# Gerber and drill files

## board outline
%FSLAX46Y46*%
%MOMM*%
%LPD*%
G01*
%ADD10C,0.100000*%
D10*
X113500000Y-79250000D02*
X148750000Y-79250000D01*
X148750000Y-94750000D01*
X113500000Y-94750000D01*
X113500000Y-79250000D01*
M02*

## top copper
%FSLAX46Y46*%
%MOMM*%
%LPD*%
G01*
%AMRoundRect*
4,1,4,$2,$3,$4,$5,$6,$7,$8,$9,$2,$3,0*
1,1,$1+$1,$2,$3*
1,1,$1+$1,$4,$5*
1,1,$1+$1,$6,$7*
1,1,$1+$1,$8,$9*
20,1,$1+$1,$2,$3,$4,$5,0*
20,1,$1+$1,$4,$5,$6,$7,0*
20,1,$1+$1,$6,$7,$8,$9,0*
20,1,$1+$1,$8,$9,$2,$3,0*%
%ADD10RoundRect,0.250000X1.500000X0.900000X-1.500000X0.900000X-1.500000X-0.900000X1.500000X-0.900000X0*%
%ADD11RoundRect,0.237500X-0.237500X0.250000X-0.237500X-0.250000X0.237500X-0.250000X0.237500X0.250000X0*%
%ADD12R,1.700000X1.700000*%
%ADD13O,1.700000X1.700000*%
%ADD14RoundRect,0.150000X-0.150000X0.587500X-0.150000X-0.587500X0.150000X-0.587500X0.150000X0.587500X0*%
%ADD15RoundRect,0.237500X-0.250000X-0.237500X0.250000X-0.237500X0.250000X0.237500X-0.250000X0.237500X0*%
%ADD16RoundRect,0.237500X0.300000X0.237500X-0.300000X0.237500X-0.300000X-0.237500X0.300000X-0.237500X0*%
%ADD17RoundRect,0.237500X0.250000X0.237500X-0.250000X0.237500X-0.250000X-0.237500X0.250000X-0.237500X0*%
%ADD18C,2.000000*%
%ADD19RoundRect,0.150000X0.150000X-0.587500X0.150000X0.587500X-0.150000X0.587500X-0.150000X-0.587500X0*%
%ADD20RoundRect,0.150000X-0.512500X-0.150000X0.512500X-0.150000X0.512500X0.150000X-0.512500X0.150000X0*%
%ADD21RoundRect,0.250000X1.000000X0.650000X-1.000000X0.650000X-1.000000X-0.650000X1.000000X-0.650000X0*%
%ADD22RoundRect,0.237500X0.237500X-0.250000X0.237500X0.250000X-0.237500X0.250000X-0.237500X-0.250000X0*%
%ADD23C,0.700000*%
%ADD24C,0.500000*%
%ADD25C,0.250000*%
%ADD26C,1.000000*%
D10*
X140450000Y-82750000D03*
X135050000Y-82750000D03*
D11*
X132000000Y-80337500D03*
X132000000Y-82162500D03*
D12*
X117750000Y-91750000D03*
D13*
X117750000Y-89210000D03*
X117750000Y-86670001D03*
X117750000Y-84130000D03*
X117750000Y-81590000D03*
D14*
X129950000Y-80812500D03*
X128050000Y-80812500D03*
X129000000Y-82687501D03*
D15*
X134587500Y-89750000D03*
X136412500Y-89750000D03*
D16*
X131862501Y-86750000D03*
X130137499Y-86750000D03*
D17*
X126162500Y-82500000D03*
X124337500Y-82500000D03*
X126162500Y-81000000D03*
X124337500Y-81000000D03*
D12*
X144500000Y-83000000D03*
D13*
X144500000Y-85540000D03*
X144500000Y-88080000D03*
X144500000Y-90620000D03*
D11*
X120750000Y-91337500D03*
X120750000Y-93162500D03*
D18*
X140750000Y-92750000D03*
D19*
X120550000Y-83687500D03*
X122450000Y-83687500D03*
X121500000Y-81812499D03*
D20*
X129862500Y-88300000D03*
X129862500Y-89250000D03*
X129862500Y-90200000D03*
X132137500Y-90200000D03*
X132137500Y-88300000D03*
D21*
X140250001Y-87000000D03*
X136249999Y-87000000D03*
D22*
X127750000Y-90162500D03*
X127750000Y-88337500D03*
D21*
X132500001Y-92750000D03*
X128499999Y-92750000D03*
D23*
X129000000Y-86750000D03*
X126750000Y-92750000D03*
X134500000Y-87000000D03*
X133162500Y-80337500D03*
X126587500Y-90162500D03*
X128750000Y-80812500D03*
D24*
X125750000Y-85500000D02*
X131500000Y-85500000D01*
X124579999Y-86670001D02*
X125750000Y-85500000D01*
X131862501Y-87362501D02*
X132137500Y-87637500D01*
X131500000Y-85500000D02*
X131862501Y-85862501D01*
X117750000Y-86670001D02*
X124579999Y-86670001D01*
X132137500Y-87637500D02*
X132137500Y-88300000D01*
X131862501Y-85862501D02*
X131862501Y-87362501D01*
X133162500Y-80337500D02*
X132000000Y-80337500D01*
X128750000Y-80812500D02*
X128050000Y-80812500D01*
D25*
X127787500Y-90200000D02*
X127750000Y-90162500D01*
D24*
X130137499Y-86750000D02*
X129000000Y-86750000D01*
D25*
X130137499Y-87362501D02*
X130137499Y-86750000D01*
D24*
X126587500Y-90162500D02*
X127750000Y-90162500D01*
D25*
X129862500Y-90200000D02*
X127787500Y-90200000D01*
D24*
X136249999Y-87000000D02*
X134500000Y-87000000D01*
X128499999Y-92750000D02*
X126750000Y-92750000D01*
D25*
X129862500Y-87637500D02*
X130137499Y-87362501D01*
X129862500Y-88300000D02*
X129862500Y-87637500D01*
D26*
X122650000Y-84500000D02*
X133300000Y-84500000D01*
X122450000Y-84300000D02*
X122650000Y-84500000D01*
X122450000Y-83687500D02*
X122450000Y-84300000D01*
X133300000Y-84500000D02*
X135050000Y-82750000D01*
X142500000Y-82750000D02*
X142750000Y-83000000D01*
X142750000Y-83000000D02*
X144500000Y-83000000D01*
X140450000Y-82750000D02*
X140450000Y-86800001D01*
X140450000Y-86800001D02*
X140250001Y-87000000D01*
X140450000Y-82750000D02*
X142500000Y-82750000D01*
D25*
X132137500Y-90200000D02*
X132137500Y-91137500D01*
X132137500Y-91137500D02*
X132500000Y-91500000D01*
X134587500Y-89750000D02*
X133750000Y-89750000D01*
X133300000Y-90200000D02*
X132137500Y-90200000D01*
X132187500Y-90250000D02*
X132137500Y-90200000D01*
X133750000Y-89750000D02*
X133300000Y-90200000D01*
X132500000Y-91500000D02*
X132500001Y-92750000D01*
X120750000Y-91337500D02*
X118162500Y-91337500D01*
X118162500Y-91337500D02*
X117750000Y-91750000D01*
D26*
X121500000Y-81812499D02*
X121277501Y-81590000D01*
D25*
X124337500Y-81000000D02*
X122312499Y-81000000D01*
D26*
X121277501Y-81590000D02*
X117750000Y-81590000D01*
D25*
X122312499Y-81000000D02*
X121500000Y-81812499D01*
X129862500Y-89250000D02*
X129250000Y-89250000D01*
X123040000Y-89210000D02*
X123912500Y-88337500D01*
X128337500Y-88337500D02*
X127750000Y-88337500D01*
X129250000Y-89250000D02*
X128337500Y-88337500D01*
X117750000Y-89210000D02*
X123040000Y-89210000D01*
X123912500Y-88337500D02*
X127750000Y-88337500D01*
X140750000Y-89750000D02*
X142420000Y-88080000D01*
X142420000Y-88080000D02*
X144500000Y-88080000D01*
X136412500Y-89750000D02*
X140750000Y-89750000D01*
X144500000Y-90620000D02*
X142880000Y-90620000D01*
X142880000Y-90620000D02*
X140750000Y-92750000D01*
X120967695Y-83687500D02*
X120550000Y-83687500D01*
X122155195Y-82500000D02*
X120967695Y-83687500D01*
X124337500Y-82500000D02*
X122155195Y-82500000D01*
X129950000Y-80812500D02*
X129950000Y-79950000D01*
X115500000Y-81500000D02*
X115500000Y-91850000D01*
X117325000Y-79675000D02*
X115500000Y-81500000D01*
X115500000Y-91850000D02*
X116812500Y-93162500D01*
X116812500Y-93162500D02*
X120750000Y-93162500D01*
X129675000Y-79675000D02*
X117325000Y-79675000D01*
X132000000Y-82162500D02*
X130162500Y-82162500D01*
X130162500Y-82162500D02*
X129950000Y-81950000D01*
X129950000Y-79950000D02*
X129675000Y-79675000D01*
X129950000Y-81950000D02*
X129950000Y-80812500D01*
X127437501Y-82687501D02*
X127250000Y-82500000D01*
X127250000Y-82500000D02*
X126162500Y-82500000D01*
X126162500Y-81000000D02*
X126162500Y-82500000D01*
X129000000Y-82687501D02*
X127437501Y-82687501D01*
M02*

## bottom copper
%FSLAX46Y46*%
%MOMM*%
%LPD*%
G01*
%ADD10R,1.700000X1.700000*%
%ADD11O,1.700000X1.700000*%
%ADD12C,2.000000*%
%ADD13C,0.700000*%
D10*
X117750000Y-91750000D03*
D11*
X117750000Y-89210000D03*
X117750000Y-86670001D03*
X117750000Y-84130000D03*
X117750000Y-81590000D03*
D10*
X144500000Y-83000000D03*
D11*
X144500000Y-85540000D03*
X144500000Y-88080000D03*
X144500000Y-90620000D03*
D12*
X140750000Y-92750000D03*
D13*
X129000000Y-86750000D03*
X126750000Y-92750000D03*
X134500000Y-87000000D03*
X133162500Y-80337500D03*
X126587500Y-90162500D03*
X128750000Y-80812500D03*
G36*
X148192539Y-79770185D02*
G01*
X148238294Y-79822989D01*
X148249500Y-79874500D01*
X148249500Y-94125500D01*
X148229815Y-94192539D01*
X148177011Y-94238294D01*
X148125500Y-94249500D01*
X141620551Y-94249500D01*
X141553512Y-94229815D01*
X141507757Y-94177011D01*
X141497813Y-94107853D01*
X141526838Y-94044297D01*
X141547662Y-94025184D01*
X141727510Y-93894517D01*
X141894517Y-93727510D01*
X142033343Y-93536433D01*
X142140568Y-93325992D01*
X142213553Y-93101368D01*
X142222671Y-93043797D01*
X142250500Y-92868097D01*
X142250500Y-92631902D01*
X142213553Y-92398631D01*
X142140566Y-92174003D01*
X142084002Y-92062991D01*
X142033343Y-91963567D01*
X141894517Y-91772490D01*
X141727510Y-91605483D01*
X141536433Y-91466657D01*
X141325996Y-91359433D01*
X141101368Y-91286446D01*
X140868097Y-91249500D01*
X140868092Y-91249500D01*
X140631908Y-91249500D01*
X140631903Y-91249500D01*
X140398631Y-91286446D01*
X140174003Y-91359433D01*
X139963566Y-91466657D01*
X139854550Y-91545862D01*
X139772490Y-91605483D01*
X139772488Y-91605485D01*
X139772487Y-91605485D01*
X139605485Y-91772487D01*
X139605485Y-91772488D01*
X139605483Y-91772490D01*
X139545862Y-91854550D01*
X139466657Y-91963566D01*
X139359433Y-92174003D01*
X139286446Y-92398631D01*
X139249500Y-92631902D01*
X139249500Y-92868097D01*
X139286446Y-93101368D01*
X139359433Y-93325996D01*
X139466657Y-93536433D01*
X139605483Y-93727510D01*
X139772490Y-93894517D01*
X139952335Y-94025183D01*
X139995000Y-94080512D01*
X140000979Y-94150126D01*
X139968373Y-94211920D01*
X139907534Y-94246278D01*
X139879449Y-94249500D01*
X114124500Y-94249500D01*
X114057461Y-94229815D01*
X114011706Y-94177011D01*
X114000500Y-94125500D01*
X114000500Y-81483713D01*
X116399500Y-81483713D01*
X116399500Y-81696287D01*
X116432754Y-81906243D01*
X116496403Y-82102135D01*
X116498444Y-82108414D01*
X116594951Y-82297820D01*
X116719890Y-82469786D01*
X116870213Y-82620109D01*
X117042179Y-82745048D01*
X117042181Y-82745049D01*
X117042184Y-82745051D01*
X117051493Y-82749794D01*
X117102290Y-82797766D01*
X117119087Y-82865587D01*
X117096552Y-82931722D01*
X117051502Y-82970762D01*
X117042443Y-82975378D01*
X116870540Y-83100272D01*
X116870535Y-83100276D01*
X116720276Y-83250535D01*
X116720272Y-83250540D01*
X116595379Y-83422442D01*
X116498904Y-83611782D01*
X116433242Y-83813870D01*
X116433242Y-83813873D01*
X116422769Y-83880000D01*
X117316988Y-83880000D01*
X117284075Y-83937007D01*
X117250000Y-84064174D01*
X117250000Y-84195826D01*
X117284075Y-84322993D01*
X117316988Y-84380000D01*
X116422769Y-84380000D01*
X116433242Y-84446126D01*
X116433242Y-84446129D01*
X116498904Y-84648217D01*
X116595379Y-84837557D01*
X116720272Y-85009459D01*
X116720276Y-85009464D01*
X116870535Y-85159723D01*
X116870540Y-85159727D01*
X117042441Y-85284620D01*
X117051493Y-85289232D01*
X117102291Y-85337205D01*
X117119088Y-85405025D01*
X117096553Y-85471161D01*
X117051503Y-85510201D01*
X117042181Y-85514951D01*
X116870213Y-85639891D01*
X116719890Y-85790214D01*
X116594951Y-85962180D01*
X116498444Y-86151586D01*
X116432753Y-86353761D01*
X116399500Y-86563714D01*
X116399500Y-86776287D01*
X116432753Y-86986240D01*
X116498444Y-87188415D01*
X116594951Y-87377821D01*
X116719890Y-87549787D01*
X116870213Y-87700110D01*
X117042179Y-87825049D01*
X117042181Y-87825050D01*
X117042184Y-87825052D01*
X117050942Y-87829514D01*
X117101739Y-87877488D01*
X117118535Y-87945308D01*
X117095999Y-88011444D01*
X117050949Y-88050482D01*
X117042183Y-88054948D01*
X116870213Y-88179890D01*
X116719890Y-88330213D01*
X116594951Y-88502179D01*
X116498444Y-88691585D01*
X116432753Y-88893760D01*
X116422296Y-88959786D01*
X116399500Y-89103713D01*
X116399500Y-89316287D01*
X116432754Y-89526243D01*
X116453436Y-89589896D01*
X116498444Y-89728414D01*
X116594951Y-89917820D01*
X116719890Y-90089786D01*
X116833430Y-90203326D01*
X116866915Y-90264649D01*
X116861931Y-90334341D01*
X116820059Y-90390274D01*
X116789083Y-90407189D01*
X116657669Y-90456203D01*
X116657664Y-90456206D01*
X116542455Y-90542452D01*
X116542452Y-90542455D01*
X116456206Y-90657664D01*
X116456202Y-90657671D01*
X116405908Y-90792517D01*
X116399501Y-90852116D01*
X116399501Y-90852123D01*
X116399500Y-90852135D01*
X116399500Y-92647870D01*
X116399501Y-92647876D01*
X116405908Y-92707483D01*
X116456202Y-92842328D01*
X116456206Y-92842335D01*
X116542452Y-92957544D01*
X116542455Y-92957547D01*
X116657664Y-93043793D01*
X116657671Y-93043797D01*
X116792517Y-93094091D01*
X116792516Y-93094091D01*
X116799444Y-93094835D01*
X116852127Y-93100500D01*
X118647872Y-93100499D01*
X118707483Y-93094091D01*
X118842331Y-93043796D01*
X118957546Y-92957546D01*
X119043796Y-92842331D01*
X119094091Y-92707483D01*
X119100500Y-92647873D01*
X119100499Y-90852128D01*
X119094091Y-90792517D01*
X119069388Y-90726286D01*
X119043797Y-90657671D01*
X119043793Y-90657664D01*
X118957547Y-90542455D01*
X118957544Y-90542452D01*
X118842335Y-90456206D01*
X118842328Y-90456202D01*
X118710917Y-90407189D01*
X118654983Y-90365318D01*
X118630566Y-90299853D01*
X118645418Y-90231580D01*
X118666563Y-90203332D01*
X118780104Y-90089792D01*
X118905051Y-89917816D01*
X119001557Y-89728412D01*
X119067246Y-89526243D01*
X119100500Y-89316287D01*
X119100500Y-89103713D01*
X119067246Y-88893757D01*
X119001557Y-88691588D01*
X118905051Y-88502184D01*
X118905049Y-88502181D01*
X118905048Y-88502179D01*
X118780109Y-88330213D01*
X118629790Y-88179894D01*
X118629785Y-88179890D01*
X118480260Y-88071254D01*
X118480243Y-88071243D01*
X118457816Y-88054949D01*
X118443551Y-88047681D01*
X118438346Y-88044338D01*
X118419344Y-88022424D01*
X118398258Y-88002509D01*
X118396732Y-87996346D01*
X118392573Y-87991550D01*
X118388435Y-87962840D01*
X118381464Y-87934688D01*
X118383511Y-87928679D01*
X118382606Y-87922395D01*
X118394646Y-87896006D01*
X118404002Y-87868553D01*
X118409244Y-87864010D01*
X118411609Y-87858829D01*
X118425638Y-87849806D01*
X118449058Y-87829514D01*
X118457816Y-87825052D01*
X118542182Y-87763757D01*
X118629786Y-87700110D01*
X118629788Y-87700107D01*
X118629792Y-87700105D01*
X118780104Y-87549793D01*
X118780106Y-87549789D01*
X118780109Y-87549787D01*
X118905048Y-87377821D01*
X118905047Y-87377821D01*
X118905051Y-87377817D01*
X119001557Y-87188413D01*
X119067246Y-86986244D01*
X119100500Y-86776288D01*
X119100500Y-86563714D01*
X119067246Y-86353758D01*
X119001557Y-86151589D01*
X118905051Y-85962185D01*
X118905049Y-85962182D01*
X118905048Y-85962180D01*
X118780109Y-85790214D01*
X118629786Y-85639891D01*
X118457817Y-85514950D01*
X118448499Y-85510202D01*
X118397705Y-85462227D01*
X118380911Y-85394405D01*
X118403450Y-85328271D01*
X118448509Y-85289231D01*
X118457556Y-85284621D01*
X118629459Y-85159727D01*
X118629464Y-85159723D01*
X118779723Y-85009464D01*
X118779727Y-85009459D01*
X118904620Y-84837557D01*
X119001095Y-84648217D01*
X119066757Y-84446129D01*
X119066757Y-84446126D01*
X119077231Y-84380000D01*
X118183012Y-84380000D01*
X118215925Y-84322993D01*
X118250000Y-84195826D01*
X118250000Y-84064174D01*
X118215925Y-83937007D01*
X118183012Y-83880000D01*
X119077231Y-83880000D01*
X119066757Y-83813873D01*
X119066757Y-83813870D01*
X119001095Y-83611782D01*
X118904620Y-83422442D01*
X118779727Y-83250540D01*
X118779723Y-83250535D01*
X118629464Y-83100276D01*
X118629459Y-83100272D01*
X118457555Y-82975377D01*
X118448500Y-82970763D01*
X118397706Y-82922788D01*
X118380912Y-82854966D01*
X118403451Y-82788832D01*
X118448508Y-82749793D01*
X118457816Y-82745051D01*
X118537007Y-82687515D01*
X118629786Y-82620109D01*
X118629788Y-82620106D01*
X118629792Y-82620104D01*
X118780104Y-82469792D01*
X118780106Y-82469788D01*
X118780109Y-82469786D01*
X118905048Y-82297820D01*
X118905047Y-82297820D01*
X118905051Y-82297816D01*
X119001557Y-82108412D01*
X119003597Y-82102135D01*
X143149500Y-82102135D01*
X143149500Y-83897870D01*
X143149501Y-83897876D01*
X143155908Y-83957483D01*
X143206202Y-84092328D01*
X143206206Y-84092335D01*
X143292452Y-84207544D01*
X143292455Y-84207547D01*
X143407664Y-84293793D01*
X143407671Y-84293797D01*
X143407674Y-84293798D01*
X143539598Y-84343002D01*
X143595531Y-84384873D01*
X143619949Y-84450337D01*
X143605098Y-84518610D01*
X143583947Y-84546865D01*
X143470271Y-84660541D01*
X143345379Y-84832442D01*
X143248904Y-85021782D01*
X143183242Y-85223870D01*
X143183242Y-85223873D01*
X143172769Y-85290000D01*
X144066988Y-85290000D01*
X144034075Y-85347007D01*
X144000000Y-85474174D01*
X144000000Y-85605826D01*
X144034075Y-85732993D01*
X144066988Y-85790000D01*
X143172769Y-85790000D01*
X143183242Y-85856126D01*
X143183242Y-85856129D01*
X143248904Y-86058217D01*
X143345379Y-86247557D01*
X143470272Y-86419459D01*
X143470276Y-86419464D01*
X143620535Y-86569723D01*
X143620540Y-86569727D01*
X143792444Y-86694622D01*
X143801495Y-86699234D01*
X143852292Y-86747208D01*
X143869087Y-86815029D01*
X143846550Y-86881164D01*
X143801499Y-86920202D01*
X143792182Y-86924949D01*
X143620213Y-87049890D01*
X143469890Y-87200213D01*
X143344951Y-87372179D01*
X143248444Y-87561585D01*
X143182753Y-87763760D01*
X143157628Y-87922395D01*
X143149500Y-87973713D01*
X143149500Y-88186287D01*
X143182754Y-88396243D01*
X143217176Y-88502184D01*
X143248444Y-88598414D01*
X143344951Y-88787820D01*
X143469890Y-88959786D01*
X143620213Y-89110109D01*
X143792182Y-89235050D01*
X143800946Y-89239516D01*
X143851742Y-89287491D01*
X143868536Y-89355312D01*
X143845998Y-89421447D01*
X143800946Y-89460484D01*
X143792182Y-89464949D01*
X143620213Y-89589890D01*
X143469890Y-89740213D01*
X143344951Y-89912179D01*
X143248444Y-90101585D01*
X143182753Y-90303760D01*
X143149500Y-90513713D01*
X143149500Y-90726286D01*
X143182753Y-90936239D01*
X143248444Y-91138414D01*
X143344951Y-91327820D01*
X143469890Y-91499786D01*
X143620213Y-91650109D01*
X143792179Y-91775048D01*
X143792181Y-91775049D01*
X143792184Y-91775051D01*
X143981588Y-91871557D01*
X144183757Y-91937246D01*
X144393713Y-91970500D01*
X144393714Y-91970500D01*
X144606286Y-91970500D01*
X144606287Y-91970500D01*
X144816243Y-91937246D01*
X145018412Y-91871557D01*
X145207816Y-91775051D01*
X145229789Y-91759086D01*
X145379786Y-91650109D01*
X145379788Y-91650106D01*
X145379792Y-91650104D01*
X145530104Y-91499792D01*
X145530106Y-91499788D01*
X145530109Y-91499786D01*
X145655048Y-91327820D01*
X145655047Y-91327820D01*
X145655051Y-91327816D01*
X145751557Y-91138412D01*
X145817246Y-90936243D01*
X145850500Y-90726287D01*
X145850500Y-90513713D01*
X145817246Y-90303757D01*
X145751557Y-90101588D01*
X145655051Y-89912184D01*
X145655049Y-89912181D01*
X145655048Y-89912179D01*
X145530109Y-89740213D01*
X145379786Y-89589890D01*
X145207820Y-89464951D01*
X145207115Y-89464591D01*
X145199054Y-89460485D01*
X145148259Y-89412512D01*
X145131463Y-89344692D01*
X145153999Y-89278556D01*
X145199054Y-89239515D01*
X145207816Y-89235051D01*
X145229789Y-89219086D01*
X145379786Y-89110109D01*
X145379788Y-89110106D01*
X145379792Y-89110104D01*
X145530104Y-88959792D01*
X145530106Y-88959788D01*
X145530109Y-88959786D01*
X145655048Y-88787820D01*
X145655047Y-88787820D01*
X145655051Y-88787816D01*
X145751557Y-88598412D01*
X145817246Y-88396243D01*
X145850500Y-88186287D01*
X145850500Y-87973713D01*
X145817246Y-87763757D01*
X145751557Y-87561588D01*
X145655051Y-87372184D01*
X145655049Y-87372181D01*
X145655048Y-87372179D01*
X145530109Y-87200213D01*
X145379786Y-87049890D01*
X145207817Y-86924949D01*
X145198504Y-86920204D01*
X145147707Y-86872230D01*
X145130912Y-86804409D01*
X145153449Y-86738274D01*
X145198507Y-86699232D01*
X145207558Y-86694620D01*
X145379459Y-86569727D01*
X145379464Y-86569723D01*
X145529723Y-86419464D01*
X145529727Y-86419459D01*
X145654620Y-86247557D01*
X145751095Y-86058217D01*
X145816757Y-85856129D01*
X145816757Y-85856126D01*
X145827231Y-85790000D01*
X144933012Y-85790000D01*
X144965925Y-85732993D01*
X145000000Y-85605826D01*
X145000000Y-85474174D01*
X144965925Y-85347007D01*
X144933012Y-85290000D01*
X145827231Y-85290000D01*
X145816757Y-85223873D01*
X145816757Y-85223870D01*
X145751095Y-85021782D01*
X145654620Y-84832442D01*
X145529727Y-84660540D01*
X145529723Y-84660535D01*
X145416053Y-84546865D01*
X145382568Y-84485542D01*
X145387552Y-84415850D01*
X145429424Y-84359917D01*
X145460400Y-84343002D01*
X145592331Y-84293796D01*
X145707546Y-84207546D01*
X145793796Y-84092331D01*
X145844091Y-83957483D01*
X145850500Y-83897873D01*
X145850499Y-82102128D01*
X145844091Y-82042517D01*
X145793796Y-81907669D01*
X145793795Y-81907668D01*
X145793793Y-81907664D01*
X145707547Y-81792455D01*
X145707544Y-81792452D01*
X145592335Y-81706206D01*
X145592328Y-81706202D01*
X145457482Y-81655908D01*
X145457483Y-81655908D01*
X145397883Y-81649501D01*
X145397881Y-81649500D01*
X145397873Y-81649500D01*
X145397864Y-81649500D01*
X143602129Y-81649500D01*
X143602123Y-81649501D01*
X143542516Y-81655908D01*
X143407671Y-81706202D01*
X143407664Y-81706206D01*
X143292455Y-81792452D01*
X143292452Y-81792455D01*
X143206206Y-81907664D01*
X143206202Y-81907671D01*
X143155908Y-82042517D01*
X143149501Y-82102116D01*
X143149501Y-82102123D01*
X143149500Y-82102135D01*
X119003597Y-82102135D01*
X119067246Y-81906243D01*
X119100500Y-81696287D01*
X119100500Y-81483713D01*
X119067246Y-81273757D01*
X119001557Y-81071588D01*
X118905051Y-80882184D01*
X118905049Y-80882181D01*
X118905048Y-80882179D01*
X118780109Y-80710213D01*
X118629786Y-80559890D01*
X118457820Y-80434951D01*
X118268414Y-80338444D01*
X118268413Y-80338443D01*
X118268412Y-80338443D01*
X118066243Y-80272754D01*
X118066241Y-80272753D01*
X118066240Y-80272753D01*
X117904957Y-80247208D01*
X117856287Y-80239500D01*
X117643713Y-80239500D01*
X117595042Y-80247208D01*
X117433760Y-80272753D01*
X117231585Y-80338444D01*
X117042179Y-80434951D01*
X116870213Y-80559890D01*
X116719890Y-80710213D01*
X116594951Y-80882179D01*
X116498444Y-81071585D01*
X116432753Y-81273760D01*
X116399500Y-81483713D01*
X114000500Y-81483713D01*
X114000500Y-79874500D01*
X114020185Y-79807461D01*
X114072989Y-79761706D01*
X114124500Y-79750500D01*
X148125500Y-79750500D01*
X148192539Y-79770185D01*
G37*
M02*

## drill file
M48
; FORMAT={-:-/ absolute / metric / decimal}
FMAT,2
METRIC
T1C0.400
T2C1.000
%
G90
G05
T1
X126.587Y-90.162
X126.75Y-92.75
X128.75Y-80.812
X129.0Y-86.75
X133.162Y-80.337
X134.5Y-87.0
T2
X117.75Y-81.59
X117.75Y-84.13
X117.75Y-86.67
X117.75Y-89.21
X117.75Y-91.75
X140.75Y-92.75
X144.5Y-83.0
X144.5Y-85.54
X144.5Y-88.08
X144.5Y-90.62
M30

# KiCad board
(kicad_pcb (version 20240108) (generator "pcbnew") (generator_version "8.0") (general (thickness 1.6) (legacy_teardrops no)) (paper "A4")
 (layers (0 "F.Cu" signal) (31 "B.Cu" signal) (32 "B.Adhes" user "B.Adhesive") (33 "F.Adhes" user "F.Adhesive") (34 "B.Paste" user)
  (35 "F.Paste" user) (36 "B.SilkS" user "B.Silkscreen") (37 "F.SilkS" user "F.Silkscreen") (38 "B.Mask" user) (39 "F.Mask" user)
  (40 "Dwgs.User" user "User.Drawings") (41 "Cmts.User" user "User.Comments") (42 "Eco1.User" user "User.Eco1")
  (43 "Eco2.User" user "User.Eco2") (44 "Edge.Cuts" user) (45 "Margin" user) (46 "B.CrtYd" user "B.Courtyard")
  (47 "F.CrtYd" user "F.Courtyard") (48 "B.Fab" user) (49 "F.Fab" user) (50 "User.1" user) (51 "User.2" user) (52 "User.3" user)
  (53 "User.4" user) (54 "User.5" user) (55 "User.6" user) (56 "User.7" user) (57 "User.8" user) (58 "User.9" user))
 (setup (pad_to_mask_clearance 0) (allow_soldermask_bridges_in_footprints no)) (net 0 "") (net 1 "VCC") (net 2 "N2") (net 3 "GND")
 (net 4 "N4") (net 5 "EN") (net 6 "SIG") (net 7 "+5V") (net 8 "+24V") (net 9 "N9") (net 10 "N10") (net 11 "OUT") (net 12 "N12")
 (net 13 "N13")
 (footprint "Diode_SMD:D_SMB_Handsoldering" (layer "F.Cu") (at 137.75 82.75 180)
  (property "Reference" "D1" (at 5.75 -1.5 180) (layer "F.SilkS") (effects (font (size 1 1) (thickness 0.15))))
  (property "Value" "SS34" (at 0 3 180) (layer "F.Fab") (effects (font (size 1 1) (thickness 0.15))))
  (pad "1" smd roundrect (at -2.7 0 180) (size 3.5 2.3) (layers "F.Cu" "F.Paste" "F.Mask") (roundrect_rratio 0.1086956522) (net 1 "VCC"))
  (pad "2" smd roundrect (at 2.7 0 180) (size 3.5 2.3) (layers "F.Cu" "F.Paste" "F.Mask") (roundrect_rratio 0.1086956522) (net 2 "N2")))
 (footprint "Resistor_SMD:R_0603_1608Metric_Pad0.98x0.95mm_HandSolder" (layer "F.Cu") (at 132 81.25 -90)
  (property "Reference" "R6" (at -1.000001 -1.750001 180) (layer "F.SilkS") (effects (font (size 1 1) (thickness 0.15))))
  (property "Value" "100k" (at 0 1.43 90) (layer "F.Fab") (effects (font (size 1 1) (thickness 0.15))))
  (pad "1" smd roundrect (at -0.9125 0 270) (size 0.975 0.95) (layers "F.Cu" "F.Paste" "F.Mask") (roundrect_rratio 0.25) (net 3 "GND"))
  (pad "2" smd roundrect (at 0.9125 0 270) (size 0.975 0.95) (layers "F.Cu" "F.Paste" "F.Mask") (roundrect_rratio 0.25) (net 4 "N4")))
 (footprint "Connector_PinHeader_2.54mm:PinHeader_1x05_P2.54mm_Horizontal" (layer "F.Cu") (at 117.75 91.75 180)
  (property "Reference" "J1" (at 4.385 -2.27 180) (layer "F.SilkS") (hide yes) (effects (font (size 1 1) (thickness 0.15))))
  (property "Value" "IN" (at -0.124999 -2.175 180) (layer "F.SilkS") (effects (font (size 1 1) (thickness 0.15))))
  (pad "1" thru_hole rect (at 0 0 180) (size 1.7 1.7) (drill 1) (layers "*.Cu" "*.Mask") (remove_unused_layers no) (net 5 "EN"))
  (pad "2" thru_hole oval (at 0 2.54 180) (size 1.7 1.7) (drill 1) (layers "*.Cu" "*.Mask") (remove_unused_layers no) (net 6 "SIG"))
  (pad "3" thru_hole oval (at 0 5.079999 180) (size 1.7 1.7) (drill 1) (layers "*.Cu" "*.Mask") (remove_unused_layers no) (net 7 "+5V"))
  (pad "4" thru_hole oval (at 0 7.62 180) (size 1.7 1.7) (drill 1) (layers "*.Cu" "*.Mask") (remove_unused_layers no) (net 3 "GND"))
  (pad "5" thru_hole oval (at 0 10.16 180) (size 1.7 1.7) (drill 1) (layers "*.Cu" "*.Mask") (remove_unused_layers no) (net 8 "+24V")))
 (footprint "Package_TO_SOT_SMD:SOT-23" (layer "F.Cu") (at 129 81.75 -90)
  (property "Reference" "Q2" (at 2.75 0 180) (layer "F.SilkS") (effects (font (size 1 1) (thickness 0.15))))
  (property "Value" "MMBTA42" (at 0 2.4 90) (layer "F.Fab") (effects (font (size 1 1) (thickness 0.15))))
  (pad "1" smd roundrect (at -0.9375 -0.95 270) (size 1.475 0.6) (layers "F.Cu" "F.Paste" "F.Mask") (roundrect_rratio 0.25) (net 4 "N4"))
  (pad "2" smd roundrect (at -0.9375 0.95 270) (size 1.475 0.6) (layers "F.Cu" "F.Paste" "F.Mask") (roundrect_rratio 0.25) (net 3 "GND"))
  (pad "3" smd roundrect (at 0.937501 0 270) (size 1.475 0.6) (layers "F.Cu" "F.Paste" "F.Mask") (roundrect_rratio 0.25) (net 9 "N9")))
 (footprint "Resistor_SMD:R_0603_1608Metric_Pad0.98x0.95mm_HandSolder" (layer "F.Cu") (at 135.5 89.75)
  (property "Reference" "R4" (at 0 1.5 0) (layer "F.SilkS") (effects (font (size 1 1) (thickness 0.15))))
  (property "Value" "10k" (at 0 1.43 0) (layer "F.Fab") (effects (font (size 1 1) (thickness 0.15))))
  (pad "1" smd roundrect (at -0.9125 0) (size 0.975 0.95) (layers "F.Cu" "F.Paste" "F.Mask") (roundrect_rratio 0.25) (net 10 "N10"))
  (pad "2" smd roundrect (at 0.9125 0) (size 0.975 0.95) (layers "F.Cu" "F.Paste" "F.Mask") (roundrect_rratio 0.25) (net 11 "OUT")))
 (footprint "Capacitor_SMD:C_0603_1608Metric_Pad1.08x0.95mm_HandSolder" (layer "F.Cu") (at 131 86.75 180)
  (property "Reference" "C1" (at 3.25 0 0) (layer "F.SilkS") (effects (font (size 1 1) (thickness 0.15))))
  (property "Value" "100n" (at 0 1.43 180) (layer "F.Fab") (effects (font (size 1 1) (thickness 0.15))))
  (pad "1" smd roundrect (at -0.862501 0 180) (size 1.075 0.95) (layers "F.Cu" "F.Paste" "F.Mask") (roundrect_rratio 0.25) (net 7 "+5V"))
  (pad "2" smd roundrect (at 0.862501 0 180) (size 1.075 0.95) (layers "F.Cu" "F.Paste" "F.Mask") (roundrect_rratio 0.25) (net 3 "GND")))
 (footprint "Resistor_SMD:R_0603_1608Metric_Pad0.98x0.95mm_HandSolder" (layer "F.Cu") (at 125.25 82.5 180)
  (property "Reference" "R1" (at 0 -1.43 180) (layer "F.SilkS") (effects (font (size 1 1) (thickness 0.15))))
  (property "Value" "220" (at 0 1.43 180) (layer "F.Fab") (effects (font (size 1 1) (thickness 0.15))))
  (pad "1" smd roundrect (at -0.9125 0 180) (size 0.975 0.95) (layers "F.Cu" "F.Paste" "F.Mask") (roundrect_rratio 0.25) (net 9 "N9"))
  (pad "2" smd roundrect (at 0.9125 0 180) (size 0.975 0.95) (layers "F.Cu" "F.Paste" "F.Mask") (roundrect_rratio 0.25) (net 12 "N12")))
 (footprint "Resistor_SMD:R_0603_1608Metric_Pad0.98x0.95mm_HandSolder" (layer "F.Cu") (at 125.25 81 180)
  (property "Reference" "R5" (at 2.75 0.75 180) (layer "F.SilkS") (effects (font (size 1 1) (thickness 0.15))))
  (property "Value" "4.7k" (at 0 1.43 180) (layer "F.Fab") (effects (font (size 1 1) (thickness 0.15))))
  (pad "1" smd roundrect (at -0.9125 0 180) (size 0.975 0.95) (layers "F.Cu" "F.Paste" "F.Mask") (roundrect_rratio 0.25) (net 9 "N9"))
  (pad "2" smd roundrect (at 0.9125 0 180) (size 0.975 0.95) (layers "F.Cu" "F.Paste" "F.Mask") (roundrect_rratio 0.25) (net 8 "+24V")))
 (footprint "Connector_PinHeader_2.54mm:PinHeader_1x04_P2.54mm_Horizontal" (layer "F.Cu") (at 144.5 83)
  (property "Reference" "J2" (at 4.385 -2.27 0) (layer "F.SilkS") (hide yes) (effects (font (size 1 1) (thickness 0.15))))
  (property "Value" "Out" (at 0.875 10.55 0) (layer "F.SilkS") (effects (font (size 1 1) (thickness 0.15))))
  (pad "1" thru_hole rect (at 0 0) (size 1.7 1.7) (drill 1) (layers "*.Cu" "*.Mask") (remove_unused_layers no) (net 1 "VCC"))
  (pad "2" thru_hole oval (at 0 2.54) (size 1.7 1.7) (drill 1) (layers "*.Cu" "*.Mask") (remove_unused_layers no) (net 3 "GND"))
  (pad "3" thru_hole oval (at 0 5.08) (size 1.7 1.7) (drill 1) (layers "*.Cu" "*.Mask") (remove_unused_layers no) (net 11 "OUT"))
  (pad "4" thru_hole oval (at 0 7.62) (size 1.7 1.7) (drill 1) (layers "*.Cu" "*.Mask") (remove_unused_layers no) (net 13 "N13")))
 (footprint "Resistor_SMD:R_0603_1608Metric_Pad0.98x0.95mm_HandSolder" (layer "F.Cu") (at 120.75 92.25 -90)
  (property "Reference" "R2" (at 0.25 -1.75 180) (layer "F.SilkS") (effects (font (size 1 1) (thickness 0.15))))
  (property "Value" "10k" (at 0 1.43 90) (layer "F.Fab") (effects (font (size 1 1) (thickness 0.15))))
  (pad "1" smd roundrect (at -0.9125 0 270) (size 0.975 0.95) (layers "F.Cu" "F.Paste" "F.Mask") (roundrect_rratio 0.25) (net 5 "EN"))
  (pad "2" smd roundrect (at 0.9125 0 270) (size 0.975 0.95) (layers "F.Cu" "F.Paste" "F.Mask") (roundrect_rratio 0.25) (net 4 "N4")))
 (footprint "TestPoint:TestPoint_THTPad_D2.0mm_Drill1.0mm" (layer "F.Cu") (at 140.75 92.75)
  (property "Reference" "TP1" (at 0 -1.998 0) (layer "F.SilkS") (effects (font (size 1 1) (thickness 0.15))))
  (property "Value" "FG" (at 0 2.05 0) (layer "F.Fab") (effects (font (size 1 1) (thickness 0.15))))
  (pad "1" thru_hole circle (at 0 0) (size 2 2) (drill 1) (layers "*.Cu" "*.Mask") (remove_unused_layers no) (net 13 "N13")))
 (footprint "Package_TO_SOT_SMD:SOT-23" (layer "F.Cu") (at 121.5 82.75 90)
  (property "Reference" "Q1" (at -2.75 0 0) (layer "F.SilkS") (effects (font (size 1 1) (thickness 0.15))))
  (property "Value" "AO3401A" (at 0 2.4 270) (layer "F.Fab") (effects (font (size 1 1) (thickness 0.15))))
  (pad "1" smd roundrect (at -0.9375 -0.95 90) (size 1.475 0.6) (layers "F.Cu" "F.Paste" "F.Mask") (roundrect_rratio 0.25) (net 12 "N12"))
  (pad "2" smd roundrect (at -0.9375 0.95 90) (size 1.475 0.6) (layers "F.Cu" "F.Paste" "F.Mask") (roundrect_rratio 0.25) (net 2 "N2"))
  (pad "3" smd roundrect (at 0.937501 0 90) (size 1.475 0.6) (layers "F.Cu" "F.Paste" "F.Mask") (roundrect_rratio 0.25) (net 8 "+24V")))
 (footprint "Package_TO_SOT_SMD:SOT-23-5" (layer "F.Cu") (at 131 89.25)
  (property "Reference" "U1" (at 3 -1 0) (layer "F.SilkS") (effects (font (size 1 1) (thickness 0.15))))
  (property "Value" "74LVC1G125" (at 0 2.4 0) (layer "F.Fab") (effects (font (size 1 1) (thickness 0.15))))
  (pad "1" smd roundrect (at -1.1375 -0.95) (size 1.325 0.6) (layers "F.Cu" "F.Paste" "F.Mask") (roundrect_rratio 0.25) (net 3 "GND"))
  (pad "2" smd roundrect (at -1.1375 0) (size 1.325 0.6) (layers "F.Cu" "F.Paste" "F.Mask") (roundrect_rratio 0.25) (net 6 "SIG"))
  (pad "3" smd roundrect (at -1.1375 0.95) (size 1.325 0.6) (layers "F.Cu" "F.Paste" "F.Mask") (roundrect_rratio 0.25) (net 3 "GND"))
  (pad "4" smd roundrect (at 1.1375 0.95) (size 1.325 0.6) (layers "F.Cu" "F.Paste" "F.Mask") (roundrect_rratio 0.25) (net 10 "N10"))
  (pad "5" smd roundrect (at 1.1375 -0.95) (size 1.325 0.6) (layers "F.Cu" "F.Paste" "F.Mask") (roundrect_rratio 0.25) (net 7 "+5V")))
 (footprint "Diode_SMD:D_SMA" (layer "F.Cu") (at 138.25 87 180)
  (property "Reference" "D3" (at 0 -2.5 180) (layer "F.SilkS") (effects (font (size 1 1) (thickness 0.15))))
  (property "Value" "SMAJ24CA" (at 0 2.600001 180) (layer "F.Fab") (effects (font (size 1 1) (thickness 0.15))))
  (pad "1" smd roundrect (at -2.000001 0 180) (size 2.5 1.8) (layers "F.Cu" "F.Paste" "F.Mask") (roundrect_rratio 0.1388888889)
   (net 1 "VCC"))
  (pad "2" smd roundrect (at 2.000001 0 180) (size 2.5 1.8) (layers "F.Cu" "F.Paste" "F.Mask") (roundrect_rratio 0.1388888889) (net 3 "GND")))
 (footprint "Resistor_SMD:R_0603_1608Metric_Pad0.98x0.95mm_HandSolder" (layer "F.Cu") (at 127.75 89.25 90)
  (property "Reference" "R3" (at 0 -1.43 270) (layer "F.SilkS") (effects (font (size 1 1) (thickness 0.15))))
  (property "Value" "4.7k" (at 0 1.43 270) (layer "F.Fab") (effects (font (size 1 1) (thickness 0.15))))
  (pad "1" smd roundrect (at -0.9125 0 90) (size 0.975 0.95) (layers "F.Cu" "F.Paste" "F.Mask") (roundrect_rratio 0.25) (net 3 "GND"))
  (pad "2" smd roundrect (at 0.9125 0 90) (size 0.975 0.95) (layers "F.Cu" "F.Paste" "F.Mask") (roundrect_rratio 0.25) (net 6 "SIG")))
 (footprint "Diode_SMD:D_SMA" (layer "F.Cu") (at 130.5 92.75 180)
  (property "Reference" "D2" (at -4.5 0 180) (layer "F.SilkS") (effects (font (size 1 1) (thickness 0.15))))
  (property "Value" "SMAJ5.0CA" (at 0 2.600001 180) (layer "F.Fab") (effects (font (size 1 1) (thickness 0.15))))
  (pad "1" smd roundrect (at -2.000001 0 180) (size 2.5 1.8) (layers "F.Cu" "F.Paste" "F.Mask") (roundrect_rratio 0.1388888889)
   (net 10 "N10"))
  (pad "2" smd roundrect (at 2.000001 0 180) (size 2.5 1.8) (layers "F.Cu" "F.Paste" "F.Mask") (roundrect_rratio 0.1388888889) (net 3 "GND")))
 (gr_rect (start 113.5 79.25) (end 148.75 94.75) (stroke (width 0.1) (type default)) (fill none) (layer "Edge.Cuts"))
 (segment (start 125.75 85.5) (end 131.5 85.5) (width 0.5) (layer "F.Cu") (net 7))
 (segment (start 124.579999 86.670001) (end 125.75 85.5) (width 0.5) (layer "F.Cu") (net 7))
 (segment (start 131.862501 87.362501) (end 132.1375 87.6375) (width 0.5) (layer "F.Cu") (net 7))
 (segment (start 131.5 85.5) (end 131.862501 85.862501) (width 0.5) (layer "F.Cu") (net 7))
 (segment (start 117.75 86.670001) (end 124.579999 86.670001) (width 0.5) (layer "F.Cu") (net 7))
 (segment (start 132.1375 87.6375) (end 132.1375 88.3) (width 0.5) (layer "F.Cu") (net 7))
 (segment (start 131.862501 85.862501) (end 131.862501 87.362501) (width 0.5) (layer "F.Cu") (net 7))
 (segment (start 133.1625 80.3375) (end 132 80.3375) (width 0.5) (layer "F.Cu") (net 3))
 (segment (start 128.75 80.8125) (end 128.05 80.8125) (width 0.5) (layer "F.Cu") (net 3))
 (segment (start 127.7875 90.2) (end 127.75 90.1625) (width 0.25) (layer "F.Cu") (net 3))
 (segment (start 130.137499 86.75) (end 129 86.75) (width 0.5) (layer "F.Cu") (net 3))
 (segment (start 130.137499 87.362501) (end 130.137499 86.75) (width 0.25) (layer "F.Cu") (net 3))
 (segment (start 126.5875 90.1625) (end 127.75 90.1625) (width 0.5) (layer "F.Cu") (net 3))
 (segment (start 129.8625 90.2) (end 127.7875 90.2) (width 0.25) (layer "F.Cu") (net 3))
 (segment (start 136.249999 87) (end 134.5 87) (width 0.5) (layer "F.Cu") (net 3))
 (segment (start 128.499999 92.75) (end 126.75 92.75) (width 0.5) (layer "F.Cu") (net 3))
 (segment (start 129.8625 87.6375) (end 130.137499 87.362501) (width 0.25) (layer "F.Cu") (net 3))
 (segment (start 129.8625 88.3) (end 129.8625 87.6375) (width 0.25) (layer "F.Cu") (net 3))
 (via (at 129 86.75) (size 0.7) (drill 0.4) (layers "F.Cu" "B.Cu") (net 3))
 (via (at 126.75 92.75) (size 0.7) (drill 0.4) (layers "F.Cu" "B.Cu") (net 3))
 (via (at 134.5 87) (size 0.7) (drill 0.4) (layers "F.Cu" "B.Cu") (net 3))
 (via (at 133.1625 80.3375) (size 0.7) (drill 0.4) (layers "F.Cu" "B.Cu") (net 3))
 (via (at 126.5875 90.1625) (size 0.7) (drill 0.4) (layers "F.Cu" "B.Cu") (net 3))
 (via (at 128.75 80.8125) (size 0.7) (drill 0.4) (layers "F.Cu" "B.Cu") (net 3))
 (segment (start 122.65 84.5) (end 133.3 84.5) (width 1) (layer "F.Cu") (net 2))
 (segment (start 122.45 84.3) (end 122.65 84.5) (width 1) (layer "F.Cu") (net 2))
 (segment (start 122.45 83.6875) (end 122.45 84.3) (width 1) (layer "F.Cu") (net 2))
 (segment (start 133.3 84.5) (end 135.05 82.75) (width 1) (layer "F.Cu") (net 2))
 (segment (start 142.5 82.75) (end 142.75 83) (width 1) (layer "F.Cu") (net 1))
 (segment (start 142.75 83) (end 144.5 83) (width 1) (layer "F.Cu") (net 1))
 (segment (start 140.45 82.75) (end 140.45 86.800001) (width 1) (layer "F.Cu") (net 1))
 (segment (start 140.45 86.800001) (end 140.250001 87) (width 1) (layer "F.Cu") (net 1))
 (segment (start 140.45 82.75) (end 142.5 82.75) (width 1) (layer "F.Cu") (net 1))
 (segment (start 132.1375 90.2) (end 132.1375 91.1375) (width 0.25) (layer "F.Cu") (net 10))
 (segment (start 132.1375 91.1375) (end 132.5 91.5) (width 0.25) (layer "F.Cu") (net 10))
 (segment (start 134.5875 89.75) (end 133.75 89.75) (width 0.25) (layer "F.Cu") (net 10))
 (segment (start 133.3 90.2) (end 132.1375 90.2) (width 0.25) (layer "F.Cu") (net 10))
 (segment (start 132.1875 90.25) (end 132.1375 90.2) (width 0.25) (layer "F.Cu") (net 10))
 (segment (start 133.75 89.75) (end 133.3 90.2) (width 0.25) (layer "F.Cu") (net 10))
 (segment (start 132.5 91.5) (end 132.500001 92.75) (width 0.25) (layer "F.Cu") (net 10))
 (segment (start 120.75 91.3375) (end 118.1625 91.3375) (width 0.25) (layer "F.Cu") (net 5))
 (segment (start 118.1625 91.3375) (end 117.75 91.75) (width 0.25) (layer "F.Cu") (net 5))
 (segment (start 121.5 81.812499) (end 121.277501 81.59) (width 1) (layer "F.Cu") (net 8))
 (segment (start 124.3375 81) (end 122.312499 81) (width 0.25) (layer "F.Cu") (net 8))
 (segment (start 121.277501 81.59) (end 117.75 81.59) (width 1) (layer "F.Cu") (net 8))
 (segment (start 122.312499 81) (end 121.5 81.812499) (width 0.25) (layer "F.Cu") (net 8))
 (segment (start 129.8625 89.25) (end 129.25 89.25) (width 0.25) (layer "F.Cu") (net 6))
 (segment (start 123.04 89.21) (end 123.9125 88.3375) (width 0.25) (layer "F.Cu") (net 6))
 (segment (start 128.3375 88.3375) (end 127.75 88.3375) (width 0.25) (layer "F.Cu") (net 6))
 (segment (start 129.25 89.25) (end 128.3375 88.3375) (width 0.25) (layer "F.Cu") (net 6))
 (segment (start 117.75 89.21) (end 123.04 89.21) (width 0.25) (layer "F.Cu") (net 6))
 (segment (start 123.9125 88.3375) (end 127.75 88.3375) (width 0.25) (layer "F.Cu") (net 6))
 (segment (start 140.75 89.75) (end 142.42 88.08) (width 0.25) (layer "F.Cu") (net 11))
 (segment (start 142.42 88.08) (end 144.5 88.08) (width 0.25) (layer "F.Cu") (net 11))
 (segment (start 136.4125 89.75) (end 140.75 89.75) (width 0.25) (layer "F.Cu") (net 11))
 (segment (start 144.5 90.62) (end 142.88 90.62) (width 0.25) (layer "F.Cu") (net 13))
 (segment (start 142.88 90.62) (end 140.75 92.75) (width 0.25) (layer "F.Cu") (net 13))
 (segment (start 120.967695 83.6875) (end 120.55 83.6875) (width 0.25) (layer "F.Cu") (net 12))
 (segment (start 122.155195 82.5) (end 120.967695 83.6875) (width 0.25) (layer "F.Cu") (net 12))
 (segment (start 124.3375 82.5) (end 122.155195 82.5) (width 0.25) (layer "F.Cu") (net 12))
 (segment (start 129.95 80.8125) (end 129.95 79.95) (width 0.25) (layer "F.Cu") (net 4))
 (segment (start 115.5 81.5) (end 115.5 91.85) (width 0.25) (layer "F.Cu") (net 4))
 (segment (start 117.325 79.675) (end 115.5 81.5) (width 0.25) (layer "F.Cu") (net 4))
 (segment (start 115.5 91.85) (end 116.8125 93.1625) (width 0.25) (layer "F.Cu") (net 4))
 (segment (start 116.8125 93.1625) (end 120.75 93.1625) (width 0.25) (layer "F.Cu") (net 4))
 (segment (start 129.675 79.675) (end 117.325 79.675) (width 0.25) (layer "F.Cu") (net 4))
 (segment (start 132 82.1625) (end 130.1625 82.1625) (width 0.25) (layer "F.Cu") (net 4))
 (segment (start 130.1625 82.1625) (end 129.95 81.95) (width 0.25) (layer "F.Cu") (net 4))
 (segment (start 129.95 79.95) (end 129.675 79.675) (width 0.25) (layer "F.Cu") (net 4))
 (segment (start 129.95 81.95) (end 129.95 80.8125) (width 0.25) (layer "F.Cu") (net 4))
 (segment (start 127.437501 82.687501) (end 127.25 82.5) (width 0.25) (layer "F.Cu") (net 9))
 (segment (start 127.25 82.5) (end 126.1625 82.5) (width 0.25) (layer "F.Cu") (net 9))
 (segment (start 126.1625 81) (end 126.1625 82.5) (width 0.25) (layer "F.Cu") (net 9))
 (segment (start 129 82.687501) (end 127.437501 82.687501) (width 0.25) (layer "F.Cu") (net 9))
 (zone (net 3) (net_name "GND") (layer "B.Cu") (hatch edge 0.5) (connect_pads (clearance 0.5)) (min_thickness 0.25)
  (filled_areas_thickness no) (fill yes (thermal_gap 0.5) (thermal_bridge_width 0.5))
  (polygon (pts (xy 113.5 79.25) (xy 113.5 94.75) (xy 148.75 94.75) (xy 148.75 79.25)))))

